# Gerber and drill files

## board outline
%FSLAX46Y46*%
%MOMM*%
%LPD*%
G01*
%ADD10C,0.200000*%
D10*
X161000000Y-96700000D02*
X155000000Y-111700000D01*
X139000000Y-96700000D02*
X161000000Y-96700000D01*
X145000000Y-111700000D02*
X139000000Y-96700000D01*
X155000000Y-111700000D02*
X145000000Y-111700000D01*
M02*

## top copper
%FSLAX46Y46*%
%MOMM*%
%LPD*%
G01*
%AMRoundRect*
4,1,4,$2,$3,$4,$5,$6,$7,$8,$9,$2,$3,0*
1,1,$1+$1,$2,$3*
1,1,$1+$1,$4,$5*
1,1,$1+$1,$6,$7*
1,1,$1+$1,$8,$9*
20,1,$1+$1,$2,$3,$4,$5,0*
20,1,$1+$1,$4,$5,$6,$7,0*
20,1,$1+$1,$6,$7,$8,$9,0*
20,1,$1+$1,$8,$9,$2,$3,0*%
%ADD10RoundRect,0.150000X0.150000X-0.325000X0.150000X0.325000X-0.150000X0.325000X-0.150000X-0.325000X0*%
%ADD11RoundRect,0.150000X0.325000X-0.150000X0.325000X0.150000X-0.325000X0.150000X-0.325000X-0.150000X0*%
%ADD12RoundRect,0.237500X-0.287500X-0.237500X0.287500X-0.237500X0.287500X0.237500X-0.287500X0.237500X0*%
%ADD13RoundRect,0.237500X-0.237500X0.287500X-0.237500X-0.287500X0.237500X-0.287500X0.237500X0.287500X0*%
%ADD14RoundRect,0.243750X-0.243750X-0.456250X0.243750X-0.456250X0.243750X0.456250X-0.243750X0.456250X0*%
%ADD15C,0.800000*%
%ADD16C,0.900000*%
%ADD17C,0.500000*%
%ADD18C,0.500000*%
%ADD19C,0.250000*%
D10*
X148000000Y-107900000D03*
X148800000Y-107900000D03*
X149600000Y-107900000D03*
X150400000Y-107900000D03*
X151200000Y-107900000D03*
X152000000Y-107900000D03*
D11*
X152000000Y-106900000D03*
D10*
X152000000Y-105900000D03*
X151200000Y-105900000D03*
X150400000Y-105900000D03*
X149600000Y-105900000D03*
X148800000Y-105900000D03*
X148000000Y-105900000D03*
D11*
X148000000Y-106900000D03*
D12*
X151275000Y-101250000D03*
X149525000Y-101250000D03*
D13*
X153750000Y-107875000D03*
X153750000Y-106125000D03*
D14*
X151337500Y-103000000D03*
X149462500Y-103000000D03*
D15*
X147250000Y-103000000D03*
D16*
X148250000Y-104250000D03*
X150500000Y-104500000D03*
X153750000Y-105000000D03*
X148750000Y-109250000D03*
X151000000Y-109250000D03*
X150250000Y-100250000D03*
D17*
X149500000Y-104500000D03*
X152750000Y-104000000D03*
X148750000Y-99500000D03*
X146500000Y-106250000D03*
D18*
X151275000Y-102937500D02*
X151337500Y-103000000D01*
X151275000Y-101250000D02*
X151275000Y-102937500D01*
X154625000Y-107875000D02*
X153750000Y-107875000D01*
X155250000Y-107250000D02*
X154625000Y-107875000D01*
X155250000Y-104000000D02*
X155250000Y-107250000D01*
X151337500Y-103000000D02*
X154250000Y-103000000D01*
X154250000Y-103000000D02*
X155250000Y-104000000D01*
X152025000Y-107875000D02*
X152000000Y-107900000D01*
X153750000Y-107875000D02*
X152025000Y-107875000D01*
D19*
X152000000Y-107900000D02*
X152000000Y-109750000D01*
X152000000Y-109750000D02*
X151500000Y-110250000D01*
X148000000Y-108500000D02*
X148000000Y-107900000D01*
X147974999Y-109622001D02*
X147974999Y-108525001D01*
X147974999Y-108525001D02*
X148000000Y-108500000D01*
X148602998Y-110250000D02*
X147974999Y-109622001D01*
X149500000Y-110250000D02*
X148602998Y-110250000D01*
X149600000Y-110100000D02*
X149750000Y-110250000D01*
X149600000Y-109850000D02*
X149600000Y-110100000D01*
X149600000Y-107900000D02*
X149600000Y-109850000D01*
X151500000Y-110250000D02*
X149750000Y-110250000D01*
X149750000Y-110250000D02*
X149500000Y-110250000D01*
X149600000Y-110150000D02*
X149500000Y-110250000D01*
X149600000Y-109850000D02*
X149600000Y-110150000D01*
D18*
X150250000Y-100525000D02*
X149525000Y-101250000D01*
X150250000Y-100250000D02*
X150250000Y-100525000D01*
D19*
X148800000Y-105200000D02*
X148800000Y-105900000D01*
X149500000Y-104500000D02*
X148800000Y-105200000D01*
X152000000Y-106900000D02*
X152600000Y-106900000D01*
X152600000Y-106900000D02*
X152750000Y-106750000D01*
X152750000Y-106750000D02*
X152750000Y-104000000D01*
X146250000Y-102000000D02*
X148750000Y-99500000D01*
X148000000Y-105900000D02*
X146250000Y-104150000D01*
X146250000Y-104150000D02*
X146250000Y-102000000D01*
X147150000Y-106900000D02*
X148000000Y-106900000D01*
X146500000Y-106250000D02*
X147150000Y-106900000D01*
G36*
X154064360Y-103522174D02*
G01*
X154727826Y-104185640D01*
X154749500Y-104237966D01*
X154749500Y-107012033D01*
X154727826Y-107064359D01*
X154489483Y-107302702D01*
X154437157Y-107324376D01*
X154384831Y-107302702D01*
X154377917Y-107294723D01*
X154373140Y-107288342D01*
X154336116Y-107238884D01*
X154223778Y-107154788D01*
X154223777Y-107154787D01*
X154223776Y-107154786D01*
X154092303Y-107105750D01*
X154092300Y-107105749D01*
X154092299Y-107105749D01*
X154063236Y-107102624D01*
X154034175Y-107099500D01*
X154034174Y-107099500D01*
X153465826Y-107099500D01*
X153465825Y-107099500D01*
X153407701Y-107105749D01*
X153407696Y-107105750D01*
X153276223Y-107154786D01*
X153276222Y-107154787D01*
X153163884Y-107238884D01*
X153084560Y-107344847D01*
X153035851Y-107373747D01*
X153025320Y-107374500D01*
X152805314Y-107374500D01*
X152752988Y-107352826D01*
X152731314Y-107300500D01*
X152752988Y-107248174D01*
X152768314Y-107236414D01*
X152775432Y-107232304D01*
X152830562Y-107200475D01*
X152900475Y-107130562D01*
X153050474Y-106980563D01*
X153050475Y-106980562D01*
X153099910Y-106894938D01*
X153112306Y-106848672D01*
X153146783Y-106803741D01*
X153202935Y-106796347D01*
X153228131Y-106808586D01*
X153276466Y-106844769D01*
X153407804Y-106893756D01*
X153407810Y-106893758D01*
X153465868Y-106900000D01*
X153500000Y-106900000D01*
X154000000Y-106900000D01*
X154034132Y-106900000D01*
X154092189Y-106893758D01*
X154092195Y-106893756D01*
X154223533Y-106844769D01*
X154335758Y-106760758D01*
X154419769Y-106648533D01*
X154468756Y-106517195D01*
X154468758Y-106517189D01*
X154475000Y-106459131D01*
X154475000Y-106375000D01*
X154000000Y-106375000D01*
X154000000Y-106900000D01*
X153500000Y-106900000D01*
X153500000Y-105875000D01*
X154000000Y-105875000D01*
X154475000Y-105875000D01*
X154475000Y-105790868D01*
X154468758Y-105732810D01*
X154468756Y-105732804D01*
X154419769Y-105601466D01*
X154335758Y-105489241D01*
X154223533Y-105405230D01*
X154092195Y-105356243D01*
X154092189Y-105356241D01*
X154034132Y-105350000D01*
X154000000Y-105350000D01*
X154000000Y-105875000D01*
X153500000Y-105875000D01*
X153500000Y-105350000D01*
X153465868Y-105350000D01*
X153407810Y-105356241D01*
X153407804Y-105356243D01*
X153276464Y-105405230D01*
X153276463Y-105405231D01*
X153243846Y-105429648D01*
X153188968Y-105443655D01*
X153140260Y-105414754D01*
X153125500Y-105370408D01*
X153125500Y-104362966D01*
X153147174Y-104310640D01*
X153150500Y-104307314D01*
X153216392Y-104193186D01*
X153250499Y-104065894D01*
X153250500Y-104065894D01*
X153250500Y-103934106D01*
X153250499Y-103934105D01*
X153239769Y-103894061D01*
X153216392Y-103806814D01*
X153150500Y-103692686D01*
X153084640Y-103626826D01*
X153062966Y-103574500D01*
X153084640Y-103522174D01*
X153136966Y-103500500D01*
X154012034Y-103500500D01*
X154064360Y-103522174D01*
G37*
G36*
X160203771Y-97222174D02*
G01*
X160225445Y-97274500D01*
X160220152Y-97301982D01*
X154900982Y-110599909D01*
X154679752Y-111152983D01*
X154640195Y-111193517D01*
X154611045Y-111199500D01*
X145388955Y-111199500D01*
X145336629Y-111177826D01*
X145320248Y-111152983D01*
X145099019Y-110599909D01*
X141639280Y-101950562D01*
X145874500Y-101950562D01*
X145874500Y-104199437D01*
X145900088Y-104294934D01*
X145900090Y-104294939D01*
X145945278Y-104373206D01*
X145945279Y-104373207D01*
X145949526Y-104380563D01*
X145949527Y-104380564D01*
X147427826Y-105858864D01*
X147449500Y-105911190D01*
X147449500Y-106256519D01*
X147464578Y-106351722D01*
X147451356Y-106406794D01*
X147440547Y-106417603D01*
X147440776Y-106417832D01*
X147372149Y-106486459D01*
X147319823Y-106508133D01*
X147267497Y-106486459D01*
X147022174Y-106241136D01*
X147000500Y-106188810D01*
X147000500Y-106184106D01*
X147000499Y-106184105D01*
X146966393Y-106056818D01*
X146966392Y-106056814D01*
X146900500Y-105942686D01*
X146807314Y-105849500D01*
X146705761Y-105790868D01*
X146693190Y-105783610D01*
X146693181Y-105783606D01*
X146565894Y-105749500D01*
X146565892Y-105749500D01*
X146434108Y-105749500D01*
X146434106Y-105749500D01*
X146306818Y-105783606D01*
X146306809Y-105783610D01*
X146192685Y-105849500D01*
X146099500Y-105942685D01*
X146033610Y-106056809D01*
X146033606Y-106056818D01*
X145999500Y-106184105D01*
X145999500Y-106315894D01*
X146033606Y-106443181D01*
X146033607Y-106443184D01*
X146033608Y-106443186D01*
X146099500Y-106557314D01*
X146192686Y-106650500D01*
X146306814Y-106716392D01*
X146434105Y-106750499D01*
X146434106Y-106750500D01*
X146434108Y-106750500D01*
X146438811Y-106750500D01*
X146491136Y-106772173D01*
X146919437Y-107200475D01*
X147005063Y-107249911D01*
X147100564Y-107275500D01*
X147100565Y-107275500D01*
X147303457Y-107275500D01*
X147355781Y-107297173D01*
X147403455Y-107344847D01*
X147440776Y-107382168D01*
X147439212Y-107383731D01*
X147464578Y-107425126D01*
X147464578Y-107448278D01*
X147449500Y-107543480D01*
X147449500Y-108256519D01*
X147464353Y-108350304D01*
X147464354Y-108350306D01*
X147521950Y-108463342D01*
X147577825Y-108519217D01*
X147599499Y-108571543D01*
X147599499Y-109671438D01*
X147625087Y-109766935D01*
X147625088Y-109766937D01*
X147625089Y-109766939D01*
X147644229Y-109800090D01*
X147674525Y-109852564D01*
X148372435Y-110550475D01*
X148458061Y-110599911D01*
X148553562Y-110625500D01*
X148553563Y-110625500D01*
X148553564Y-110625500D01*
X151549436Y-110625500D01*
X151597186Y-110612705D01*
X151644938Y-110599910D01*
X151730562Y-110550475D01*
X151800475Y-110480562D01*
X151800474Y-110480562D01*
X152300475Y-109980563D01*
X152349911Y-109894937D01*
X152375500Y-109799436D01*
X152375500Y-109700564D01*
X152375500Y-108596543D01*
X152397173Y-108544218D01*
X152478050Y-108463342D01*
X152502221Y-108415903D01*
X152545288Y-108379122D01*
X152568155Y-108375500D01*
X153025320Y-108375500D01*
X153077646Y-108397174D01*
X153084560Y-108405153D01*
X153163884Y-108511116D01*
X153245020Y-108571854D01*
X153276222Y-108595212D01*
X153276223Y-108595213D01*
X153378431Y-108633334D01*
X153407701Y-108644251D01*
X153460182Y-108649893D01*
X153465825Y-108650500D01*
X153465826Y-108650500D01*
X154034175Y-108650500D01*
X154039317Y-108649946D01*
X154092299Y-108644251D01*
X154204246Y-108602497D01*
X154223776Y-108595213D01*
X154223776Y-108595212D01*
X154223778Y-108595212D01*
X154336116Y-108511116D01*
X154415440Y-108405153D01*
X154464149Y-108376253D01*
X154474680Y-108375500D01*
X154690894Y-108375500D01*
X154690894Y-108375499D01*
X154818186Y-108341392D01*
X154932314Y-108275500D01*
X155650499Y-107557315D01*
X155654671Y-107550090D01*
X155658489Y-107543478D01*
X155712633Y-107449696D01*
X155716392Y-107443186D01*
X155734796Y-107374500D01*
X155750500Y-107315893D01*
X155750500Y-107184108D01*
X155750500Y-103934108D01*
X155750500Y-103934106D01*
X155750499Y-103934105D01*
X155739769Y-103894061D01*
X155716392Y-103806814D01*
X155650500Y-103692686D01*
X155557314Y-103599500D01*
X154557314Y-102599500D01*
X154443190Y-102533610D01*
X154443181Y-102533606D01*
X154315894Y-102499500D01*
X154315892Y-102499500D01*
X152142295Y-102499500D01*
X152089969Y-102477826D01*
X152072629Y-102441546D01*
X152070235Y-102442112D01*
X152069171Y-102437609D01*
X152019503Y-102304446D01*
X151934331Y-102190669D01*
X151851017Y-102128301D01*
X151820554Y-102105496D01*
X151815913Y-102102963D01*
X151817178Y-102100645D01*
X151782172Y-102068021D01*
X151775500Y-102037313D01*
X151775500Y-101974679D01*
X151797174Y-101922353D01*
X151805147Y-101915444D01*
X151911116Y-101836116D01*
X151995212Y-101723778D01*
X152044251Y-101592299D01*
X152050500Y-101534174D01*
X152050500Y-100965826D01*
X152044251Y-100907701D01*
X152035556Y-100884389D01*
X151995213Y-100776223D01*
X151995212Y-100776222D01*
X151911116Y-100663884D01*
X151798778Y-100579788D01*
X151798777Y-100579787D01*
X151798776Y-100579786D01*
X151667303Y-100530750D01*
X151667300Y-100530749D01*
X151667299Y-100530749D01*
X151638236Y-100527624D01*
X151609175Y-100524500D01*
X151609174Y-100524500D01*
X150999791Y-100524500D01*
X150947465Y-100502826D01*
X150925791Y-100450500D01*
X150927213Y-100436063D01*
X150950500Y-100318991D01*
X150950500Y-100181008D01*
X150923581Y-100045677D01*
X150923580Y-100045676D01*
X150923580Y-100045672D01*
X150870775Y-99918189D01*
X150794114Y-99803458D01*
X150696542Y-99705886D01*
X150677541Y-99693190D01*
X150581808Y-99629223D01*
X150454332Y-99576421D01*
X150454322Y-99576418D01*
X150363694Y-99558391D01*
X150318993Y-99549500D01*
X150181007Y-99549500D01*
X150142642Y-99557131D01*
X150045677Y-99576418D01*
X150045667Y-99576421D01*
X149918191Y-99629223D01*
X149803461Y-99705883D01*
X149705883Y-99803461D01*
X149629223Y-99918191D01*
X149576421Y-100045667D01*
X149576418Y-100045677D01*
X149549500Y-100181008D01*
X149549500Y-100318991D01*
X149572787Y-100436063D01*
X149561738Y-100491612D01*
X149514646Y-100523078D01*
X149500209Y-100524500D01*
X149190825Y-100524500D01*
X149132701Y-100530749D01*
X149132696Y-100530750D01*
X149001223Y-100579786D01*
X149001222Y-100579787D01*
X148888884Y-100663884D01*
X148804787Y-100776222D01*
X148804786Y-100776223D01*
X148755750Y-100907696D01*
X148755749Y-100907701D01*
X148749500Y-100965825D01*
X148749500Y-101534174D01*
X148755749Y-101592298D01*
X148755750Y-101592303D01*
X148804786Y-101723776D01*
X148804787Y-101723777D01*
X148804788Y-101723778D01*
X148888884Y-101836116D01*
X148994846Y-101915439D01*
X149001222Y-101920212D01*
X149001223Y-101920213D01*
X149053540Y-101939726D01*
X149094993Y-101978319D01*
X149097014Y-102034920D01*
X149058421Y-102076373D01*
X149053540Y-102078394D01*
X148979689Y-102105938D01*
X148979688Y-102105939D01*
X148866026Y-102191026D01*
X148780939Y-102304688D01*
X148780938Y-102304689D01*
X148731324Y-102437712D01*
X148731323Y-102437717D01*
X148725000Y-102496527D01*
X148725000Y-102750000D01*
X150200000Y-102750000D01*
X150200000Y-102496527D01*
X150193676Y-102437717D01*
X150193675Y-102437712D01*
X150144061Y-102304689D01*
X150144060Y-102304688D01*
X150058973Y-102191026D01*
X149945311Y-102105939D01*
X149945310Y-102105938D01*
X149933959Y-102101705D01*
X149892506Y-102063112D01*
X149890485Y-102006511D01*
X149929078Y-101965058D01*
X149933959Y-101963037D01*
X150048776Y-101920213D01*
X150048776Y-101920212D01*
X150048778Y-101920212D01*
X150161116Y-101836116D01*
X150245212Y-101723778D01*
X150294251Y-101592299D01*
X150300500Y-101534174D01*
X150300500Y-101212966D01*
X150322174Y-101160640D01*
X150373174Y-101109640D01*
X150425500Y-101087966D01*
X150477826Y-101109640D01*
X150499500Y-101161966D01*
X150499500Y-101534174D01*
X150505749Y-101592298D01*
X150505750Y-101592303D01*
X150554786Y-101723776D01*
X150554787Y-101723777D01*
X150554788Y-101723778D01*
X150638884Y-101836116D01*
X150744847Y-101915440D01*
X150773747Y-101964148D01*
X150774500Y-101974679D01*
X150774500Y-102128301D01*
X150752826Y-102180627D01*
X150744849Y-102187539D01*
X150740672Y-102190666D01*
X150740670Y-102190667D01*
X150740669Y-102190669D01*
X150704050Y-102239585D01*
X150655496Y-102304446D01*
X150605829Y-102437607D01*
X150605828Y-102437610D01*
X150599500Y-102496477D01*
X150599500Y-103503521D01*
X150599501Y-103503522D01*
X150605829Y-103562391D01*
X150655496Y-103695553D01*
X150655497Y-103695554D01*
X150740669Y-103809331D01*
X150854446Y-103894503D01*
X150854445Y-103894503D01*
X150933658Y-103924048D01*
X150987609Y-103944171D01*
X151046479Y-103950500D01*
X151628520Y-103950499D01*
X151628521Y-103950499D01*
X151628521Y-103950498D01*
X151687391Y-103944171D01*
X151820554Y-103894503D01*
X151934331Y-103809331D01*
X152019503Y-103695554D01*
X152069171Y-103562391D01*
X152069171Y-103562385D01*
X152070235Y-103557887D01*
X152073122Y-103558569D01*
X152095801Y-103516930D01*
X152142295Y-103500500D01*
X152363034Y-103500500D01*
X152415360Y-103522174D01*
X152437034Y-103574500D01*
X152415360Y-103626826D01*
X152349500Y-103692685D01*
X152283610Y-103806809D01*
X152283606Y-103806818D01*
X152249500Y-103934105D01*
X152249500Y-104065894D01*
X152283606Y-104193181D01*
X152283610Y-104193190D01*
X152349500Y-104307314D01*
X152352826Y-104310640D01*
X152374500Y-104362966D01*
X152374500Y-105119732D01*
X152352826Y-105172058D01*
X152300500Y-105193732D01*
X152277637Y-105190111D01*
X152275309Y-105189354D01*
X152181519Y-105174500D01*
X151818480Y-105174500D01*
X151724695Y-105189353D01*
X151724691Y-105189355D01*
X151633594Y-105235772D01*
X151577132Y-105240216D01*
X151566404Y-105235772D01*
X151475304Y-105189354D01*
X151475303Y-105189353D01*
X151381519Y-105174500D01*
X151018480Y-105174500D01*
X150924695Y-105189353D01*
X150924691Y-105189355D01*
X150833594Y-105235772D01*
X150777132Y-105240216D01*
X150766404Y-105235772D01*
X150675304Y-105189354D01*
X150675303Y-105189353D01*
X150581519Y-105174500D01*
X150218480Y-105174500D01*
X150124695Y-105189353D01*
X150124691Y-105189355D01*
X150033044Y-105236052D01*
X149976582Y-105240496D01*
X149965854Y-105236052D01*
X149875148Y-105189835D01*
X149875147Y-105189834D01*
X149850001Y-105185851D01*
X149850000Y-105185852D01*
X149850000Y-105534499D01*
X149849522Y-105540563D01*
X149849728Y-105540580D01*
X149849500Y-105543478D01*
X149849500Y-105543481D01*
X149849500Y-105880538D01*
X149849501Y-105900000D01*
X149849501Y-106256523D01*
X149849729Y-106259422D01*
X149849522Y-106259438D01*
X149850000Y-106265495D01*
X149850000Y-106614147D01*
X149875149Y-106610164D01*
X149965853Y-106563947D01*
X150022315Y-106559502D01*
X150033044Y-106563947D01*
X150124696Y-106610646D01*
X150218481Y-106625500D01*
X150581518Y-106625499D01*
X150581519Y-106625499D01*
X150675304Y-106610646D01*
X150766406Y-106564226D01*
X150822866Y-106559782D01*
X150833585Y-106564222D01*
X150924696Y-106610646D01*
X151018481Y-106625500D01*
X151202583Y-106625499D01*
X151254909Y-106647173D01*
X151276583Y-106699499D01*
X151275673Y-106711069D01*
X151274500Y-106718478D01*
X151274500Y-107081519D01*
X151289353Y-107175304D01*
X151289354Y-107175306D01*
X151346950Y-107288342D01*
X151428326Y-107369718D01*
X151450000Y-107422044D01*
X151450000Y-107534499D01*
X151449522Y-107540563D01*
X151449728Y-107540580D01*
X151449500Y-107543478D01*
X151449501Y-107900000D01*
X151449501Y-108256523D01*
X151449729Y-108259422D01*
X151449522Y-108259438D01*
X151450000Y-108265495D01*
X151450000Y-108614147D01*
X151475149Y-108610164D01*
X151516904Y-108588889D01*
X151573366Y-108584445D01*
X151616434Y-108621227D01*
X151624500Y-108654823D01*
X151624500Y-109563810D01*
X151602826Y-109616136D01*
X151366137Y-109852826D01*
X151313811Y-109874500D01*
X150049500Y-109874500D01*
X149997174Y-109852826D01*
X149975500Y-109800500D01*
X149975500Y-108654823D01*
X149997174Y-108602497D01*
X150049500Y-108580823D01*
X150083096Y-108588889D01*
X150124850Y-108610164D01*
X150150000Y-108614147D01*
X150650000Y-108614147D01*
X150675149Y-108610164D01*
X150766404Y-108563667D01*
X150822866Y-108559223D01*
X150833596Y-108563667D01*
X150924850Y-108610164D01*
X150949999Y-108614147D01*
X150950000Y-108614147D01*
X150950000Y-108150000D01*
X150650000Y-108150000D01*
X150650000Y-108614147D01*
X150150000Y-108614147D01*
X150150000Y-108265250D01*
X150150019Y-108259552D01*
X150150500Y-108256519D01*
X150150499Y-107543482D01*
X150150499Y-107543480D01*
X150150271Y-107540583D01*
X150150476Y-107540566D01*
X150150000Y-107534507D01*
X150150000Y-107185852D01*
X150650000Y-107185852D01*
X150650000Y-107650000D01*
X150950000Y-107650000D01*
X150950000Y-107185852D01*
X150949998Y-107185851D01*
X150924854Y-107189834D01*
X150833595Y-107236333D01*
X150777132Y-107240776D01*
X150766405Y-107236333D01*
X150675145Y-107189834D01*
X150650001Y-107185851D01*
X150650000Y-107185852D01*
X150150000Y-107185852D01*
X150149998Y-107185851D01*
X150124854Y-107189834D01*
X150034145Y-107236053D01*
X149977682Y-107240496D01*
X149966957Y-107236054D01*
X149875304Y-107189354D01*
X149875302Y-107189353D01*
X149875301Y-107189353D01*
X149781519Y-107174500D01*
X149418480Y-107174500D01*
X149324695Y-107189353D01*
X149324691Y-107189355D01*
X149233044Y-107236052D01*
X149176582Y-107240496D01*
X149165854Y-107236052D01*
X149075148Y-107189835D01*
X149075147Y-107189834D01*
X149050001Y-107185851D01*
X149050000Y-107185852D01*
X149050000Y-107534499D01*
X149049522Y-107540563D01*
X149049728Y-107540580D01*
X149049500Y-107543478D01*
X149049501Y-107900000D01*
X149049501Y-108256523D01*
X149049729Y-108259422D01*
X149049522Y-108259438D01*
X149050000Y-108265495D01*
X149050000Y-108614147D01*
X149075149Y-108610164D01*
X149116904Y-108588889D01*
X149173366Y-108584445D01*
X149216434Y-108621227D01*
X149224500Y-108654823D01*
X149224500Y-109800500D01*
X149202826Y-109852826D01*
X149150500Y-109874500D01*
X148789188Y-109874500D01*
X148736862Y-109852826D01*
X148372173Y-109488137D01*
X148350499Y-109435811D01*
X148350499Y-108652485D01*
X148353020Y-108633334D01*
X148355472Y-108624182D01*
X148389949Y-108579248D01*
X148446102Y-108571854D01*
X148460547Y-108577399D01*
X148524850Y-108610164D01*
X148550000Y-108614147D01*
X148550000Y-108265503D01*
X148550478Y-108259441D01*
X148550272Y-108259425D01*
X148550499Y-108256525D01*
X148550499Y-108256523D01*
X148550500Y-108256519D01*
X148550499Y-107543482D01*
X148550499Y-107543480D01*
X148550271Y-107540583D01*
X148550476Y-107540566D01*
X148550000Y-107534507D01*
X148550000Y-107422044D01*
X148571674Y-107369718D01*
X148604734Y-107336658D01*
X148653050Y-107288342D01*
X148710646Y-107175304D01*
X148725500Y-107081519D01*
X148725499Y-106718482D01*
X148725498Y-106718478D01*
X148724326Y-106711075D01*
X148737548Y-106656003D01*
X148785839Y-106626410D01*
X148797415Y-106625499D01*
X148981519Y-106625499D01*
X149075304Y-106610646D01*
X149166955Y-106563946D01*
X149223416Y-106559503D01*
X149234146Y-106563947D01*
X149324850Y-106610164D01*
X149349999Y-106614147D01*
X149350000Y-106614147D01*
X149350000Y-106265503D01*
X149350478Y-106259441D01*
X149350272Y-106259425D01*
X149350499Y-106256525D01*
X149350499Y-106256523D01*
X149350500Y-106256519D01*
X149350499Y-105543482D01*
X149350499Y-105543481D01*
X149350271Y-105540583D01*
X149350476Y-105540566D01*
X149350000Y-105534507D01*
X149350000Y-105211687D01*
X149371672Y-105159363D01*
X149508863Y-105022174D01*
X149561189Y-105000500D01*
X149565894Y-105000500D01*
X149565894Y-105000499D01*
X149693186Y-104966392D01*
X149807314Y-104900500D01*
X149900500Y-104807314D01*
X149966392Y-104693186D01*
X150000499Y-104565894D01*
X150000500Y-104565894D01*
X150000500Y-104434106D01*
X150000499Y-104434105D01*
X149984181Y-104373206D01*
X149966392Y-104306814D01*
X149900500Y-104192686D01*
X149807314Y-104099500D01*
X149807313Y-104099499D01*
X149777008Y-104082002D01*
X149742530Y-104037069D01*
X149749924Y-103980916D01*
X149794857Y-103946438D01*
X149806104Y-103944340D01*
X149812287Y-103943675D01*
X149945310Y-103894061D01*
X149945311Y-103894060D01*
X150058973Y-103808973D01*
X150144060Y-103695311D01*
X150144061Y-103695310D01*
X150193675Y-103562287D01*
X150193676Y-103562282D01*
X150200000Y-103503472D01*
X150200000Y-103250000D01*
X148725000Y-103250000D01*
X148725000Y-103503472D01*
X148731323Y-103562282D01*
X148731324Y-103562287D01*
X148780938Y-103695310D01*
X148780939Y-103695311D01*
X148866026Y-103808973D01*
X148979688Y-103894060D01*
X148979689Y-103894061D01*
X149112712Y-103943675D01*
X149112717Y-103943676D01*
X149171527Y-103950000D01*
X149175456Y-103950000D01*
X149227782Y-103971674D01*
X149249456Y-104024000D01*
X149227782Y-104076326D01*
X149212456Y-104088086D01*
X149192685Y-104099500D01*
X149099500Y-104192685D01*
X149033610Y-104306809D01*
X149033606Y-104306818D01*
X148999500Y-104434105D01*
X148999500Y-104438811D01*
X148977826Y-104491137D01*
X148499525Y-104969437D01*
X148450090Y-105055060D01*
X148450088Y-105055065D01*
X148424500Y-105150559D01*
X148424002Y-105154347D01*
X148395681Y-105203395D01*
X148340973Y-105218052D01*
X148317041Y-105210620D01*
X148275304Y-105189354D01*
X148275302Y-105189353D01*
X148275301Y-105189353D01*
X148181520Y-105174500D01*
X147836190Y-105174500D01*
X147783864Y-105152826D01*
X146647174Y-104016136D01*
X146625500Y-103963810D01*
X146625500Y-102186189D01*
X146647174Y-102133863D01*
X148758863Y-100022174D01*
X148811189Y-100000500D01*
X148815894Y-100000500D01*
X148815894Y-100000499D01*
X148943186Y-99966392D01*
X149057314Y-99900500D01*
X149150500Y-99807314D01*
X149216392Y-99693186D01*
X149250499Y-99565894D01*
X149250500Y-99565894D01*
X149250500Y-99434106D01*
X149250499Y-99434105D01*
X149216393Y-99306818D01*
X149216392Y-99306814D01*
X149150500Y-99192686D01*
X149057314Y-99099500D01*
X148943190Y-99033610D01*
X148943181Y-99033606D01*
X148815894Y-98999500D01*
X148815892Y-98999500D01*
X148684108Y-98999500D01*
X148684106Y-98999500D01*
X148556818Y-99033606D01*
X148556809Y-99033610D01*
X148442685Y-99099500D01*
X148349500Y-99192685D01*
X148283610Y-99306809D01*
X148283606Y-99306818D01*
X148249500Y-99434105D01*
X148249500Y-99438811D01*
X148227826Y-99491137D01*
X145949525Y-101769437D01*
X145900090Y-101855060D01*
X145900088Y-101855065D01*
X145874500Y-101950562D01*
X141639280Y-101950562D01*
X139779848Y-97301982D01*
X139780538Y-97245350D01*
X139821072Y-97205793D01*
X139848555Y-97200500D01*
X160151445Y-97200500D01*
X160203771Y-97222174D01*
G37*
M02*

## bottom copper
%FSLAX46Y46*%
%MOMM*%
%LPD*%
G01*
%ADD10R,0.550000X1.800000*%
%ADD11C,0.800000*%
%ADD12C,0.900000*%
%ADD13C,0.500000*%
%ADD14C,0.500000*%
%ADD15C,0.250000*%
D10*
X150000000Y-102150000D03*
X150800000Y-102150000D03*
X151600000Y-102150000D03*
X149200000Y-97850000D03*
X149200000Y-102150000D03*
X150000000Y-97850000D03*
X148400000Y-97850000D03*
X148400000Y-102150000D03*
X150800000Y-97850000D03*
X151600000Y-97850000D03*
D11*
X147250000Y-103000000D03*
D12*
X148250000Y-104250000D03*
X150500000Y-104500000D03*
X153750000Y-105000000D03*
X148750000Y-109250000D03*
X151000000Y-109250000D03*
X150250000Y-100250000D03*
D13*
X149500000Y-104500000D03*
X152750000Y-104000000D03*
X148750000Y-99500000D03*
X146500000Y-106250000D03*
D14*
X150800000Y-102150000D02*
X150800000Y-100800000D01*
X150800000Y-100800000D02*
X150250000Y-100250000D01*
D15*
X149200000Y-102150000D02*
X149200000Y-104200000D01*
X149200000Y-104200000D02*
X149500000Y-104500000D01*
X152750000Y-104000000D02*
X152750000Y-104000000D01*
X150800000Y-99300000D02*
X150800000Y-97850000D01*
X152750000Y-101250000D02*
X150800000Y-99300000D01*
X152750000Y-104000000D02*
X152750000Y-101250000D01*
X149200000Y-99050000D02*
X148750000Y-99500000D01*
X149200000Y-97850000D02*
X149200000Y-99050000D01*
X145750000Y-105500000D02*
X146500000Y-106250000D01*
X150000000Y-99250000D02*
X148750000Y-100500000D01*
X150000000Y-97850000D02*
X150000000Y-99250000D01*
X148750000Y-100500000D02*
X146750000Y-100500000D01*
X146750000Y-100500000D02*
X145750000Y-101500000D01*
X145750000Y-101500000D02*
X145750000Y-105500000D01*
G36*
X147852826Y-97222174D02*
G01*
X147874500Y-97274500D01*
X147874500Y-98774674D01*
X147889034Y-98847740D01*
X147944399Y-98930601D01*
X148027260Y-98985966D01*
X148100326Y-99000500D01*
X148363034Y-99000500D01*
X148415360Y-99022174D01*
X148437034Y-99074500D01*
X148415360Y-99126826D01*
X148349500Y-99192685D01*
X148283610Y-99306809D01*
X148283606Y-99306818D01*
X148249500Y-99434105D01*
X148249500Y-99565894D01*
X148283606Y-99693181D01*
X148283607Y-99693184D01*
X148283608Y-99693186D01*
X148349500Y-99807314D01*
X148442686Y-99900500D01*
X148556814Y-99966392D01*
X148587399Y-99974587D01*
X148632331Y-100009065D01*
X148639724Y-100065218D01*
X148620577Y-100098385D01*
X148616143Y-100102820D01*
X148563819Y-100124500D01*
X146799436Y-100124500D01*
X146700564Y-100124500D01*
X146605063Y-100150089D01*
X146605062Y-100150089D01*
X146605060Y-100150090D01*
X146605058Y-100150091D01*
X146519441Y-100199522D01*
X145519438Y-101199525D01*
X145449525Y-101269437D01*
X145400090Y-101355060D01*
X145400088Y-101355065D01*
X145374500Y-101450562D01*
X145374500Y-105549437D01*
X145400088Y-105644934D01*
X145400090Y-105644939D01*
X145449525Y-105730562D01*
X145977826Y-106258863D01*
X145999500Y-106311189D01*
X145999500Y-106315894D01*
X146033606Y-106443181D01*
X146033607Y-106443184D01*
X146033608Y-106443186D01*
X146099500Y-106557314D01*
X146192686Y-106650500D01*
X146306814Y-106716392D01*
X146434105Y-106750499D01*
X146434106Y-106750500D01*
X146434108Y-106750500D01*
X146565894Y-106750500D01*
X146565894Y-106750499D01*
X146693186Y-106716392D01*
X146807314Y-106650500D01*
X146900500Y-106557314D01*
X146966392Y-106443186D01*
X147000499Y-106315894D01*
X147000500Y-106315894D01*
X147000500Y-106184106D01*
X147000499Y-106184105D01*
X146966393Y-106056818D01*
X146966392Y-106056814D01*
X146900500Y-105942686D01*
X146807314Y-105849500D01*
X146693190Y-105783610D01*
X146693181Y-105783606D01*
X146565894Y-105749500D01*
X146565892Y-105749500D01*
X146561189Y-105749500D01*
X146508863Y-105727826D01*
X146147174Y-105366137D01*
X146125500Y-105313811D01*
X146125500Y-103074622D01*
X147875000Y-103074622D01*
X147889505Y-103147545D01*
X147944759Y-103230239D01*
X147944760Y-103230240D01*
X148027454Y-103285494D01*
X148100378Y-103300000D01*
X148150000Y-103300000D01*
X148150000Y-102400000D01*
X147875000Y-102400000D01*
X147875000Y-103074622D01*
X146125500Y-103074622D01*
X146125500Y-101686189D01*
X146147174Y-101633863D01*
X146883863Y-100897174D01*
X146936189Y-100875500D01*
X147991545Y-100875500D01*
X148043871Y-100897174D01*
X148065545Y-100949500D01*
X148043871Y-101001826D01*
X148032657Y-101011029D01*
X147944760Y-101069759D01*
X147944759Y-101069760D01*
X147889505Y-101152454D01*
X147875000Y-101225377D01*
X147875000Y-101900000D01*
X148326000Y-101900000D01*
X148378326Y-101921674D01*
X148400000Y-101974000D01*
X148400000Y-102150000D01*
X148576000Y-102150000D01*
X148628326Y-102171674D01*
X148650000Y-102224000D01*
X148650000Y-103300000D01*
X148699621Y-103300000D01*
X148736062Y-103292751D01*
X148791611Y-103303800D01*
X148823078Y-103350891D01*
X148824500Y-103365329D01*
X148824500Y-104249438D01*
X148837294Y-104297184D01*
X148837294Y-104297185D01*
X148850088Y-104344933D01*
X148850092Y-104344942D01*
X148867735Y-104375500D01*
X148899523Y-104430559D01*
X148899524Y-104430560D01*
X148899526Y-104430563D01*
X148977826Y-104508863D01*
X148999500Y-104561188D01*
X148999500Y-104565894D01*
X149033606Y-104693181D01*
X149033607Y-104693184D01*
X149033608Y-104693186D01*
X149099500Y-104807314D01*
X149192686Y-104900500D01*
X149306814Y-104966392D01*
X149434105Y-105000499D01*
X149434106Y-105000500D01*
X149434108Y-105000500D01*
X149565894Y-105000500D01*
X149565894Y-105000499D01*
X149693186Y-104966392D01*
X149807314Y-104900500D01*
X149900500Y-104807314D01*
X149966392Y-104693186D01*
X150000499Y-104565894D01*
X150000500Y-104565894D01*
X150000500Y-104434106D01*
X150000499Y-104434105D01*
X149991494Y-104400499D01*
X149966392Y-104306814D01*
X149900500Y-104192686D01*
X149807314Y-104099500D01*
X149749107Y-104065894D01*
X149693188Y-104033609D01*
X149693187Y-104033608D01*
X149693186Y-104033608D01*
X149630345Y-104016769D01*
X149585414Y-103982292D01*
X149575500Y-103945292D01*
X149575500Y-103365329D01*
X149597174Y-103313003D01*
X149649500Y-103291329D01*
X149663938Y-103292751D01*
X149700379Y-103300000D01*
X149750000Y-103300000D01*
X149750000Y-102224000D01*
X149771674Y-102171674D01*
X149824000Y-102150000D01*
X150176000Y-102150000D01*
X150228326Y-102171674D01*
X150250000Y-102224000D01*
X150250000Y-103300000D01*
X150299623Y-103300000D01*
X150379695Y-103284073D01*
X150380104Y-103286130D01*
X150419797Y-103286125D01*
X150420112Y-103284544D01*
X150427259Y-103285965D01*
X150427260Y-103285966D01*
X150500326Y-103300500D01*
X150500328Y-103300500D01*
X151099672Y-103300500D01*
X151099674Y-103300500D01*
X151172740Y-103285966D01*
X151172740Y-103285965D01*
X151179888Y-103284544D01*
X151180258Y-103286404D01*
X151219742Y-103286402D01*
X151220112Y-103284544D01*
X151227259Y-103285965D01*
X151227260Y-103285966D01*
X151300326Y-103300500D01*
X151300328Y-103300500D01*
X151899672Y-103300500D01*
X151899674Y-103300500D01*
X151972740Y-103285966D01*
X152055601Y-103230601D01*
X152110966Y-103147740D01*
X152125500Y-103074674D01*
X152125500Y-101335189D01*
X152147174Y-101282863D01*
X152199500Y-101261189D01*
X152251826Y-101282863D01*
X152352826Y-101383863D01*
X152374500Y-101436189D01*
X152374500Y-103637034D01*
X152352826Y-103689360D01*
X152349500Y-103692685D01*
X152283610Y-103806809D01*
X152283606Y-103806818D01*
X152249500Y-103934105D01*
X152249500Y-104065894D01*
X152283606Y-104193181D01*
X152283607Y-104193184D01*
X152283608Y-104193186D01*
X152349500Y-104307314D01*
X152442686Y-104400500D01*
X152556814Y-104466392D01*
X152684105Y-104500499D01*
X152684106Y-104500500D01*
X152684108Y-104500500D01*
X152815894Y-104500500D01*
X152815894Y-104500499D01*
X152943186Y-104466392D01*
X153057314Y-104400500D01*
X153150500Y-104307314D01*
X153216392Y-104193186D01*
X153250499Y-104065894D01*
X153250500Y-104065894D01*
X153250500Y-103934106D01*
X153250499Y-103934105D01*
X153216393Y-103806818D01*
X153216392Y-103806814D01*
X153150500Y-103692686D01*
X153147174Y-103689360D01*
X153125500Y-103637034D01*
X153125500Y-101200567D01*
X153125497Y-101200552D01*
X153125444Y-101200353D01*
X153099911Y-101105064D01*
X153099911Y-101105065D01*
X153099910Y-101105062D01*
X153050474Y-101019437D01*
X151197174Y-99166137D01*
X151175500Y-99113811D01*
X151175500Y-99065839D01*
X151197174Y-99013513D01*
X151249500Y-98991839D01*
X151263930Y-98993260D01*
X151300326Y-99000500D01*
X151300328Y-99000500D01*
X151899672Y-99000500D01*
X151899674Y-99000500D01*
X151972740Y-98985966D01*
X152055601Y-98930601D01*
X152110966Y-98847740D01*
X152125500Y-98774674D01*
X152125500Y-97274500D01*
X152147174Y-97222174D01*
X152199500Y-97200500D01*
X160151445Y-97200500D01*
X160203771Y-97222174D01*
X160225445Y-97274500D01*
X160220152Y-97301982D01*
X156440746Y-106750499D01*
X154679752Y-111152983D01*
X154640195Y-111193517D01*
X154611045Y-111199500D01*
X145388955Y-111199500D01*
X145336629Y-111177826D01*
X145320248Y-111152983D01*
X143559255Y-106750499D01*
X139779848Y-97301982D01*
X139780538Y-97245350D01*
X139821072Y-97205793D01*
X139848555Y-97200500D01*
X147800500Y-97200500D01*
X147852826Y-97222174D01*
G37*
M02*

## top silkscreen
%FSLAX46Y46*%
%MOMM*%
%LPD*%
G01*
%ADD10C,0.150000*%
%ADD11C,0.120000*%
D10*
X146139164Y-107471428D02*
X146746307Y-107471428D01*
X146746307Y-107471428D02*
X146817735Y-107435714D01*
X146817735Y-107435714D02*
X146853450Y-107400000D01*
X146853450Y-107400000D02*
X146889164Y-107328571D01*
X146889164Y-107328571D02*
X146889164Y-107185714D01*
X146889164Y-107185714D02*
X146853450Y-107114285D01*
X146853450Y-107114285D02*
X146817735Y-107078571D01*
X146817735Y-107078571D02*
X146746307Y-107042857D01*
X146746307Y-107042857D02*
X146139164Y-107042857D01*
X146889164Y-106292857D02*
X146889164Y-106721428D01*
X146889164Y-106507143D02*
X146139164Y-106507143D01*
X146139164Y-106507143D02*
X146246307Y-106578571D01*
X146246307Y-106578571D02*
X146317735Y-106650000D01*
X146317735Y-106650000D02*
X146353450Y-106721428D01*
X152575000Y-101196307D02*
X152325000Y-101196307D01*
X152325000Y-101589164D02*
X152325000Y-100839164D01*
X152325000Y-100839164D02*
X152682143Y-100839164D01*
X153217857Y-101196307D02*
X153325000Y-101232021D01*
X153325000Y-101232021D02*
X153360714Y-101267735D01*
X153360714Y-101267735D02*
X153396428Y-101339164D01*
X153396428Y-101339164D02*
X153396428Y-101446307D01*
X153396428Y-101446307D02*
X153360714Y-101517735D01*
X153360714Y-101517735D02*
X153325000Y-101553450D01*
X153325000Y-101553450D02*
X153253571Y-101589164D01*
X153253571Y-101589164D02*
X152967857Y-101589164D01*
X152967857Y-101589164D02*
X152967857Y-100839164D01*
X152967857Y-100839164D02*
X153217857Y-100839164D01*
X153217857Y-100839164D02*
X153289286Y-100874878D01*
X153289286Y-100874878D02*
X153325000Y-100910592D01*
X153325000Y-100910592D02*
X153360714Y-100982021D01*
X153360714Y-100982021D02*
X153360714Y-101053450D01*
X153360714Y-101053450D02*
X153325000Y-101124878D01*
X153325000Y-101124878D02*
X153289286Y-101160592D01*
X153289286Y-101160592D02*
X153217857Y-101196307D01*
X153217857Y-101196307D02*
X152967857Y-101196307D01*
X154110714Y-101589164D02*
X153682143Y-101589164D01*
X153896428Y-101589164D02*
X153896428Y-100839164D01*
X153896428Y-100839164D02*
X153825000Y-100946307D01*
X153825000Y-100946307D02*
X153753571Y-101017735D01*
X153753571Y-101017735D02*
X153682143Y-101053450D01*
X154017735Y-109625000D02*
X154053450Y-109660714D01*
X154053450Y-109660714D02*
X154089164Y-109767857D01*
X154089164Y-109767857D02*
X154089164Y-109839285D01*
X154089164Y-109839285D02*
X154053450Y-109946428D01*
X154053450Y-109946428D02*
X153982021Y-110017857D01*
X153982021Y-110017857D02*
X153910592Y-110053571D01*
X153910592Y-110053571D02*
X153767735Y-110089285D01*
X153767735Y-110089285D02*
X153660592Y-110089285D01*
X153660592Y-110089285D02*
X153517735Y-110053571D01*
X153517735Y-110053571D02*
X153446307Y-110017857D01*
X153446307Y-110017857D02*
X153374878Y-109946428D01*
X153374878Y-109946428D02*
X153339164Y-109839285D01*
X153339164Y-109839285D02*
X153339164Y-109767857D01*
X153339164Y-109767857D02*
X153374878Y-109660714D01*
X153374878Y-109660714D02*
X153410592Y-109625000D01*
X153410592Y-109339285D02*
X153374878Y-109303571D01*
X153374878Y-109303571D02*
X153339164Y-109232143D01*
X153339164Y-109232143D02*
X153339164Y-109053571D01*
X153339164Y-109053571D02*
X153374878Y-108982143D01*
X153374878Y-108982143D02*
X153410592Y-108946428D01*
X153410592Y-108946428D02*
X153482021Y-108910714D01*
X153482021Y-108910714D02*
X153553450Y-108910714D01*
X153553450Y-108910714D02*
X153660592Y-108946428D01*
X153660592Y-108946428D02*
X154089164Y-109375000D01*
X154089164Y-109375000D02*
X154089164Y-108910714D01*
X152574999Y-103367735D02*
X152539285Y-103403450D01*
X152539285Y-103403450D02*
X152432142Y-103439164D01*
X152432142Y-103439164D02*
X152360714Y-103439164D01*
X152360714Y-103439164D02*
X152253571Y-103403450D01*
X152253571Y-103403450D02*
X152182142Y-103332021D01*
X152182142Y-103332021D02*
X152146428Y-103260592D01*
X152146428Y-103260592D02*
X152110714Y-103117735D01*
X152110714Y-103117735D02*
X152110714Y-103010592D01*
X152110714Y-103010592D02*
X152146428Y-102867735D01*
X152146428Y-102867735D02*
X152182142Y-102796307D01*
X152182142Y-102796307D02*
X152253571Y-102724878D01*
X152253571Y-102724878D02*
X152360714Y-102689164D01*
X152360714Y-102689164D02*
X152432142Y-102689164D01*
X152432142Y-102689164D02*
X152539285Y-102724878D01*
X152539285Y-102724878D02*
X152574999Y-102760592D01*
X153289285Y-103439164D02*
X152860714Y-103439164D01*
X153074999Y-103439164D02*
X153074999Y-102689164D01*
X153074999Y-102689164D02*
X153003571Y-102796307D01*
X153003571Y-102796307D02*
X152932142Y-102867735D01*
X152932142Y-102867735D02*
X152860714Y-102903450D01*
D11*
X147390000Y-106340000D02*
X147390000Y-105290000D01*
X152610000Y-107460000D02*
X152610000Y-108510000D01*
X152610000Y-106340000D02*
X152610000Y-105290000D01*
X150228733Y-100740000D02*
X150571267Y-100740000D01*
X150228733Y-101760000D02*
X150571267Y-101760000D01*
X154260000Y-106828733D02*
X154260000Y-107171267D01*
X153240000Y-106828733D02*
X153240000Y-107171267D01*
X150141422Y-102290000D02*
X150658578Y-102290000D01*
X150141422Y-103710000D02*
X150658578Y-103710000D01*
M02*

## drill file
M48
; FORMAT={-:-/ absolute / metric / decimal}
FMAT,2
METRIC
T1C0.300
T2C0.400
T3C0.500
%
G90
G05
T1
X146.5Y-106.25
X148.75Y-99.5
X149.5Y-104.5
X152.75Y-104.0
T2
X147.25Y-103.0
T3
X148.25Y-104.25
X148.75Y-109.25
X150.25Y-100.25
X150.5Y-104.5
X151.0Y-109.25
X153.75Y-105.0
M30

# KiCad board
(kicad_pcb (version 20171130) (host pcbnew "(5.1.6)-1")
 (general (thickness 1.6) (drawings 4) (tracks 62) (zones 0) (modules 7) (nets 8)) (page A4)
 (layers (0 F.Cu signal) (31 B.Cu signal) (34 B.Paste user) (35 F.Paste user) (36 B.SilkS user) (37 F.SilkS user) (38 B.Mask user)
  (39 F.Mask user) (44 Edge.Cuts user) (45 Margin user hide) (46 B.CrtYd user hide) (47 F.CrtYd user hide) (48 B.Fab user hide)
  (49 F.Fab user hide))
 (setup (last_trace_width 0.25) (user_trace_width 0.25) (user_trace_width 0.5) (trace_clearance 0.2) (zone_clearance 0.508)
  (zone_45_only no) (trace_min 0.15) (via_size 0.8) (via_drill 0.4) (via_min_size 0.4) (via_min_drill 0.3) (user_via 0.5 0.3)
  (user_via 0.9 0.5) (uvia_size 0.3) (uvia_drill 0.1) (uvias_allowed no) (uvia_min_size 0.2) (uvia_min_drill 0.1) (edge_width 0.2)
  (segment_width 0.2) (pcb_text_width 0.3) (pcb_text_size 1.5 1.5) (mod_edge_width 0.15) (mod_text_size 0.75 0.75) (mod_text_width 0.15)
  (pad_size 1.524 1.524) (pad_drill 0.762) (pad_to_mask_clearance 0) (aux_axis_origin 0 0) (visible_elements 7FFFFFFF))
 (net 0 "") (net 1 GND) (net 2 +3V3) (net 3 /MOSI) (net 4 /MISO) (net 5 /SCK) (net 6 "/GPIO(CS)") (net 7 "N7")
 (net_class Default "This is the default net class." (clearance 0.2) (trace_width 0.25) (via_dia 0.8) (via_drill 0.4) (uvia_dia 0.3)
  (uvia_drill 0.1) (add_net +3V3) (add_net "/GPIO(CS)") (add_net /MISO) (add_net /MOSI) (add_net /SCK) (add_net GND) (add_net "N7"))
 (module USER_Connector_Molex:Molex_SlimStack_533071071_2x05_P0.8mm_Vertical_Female (layer B.Cu) (at 150 100 180)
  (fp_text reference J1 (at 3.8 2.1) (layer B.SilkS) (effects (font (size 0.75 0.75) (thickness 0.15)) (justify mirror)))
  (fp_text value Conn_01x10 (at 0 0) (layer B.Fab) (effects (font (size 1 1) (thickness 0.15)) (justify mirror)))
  (pad 5 smd rect (at 0 -2.15) (size 0.55 1.8) (layers B.Cu B.Paste B.Mask) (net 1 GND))
  (pad 3 smd rect (at -0.8 -2.15) (size 0.55 1.8) (layers B.Cu B.Paste B.Mask) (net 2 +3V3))
  (pad 1 smd rect (at -1.6 -2.15) (size 0.55 1.8) (layers B.Cu B.Paste B.Mask))
  (pad 8 smd rect (at 0.8 2.15) (size 0.55 1.8) (layers B.Cu B.Paste B.Mask) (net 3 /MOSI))
  (pad 7 smd rect (at 0.8 -2.15) (size 0.55 1.8) (layers B.Cu B.Paste B.Mask) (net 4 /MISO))
  (pad 6 smd rect (at 0 2.15) (size 0.55 1.8) (layers B.Cu B.Paste B.Mask) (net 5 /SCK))
  (pad 10 smd rect (at 1.6 2.15) (size 0.55 1.8) (layers B.Cu B.Paste B.Mask))
  (pad 9 smd rect (at 1.6 -2.15) (size 0.55 1.8) (layers B.Cu B.Paste B.Mask) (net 1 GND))
  (pad 4 smd rect (at -0.8 2.15) (size 0.55 1.8) (layers B.Cu B.Paste B.Mask) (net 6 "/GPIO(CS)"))
  (pad 2 smd rect (at -1.6 2.15) (size 0.55 1.8) (layers B.Cu B.Paste B.Mask)))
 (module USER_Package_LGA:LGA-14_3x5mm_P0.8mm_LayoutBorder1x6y (layer F.Cu) (at 150 106.9 90)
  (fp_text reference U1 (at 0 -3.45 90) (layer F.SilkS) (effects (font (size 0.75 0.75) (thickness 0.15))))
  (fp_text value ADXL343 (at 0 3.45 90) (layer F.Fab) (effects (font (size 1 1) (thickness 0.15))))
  (fp_line (start 0.56 -2.61) (end 1.61 -2.61) (layer F.SilkS) (width 0.12))
  (fp_line (start -0.56 2.61) (end -1.61 2.61) (layer F.SilkS) (width 0.12))
  (fp_line (start 0.56 2.61) (end 1.61 2.61) (layer F.SilkS) (width 0.12))
  (pad 1 smd roundrect (at -1 -2 90) (size 0.95 0.6) (layers F.Cu F.Paste F.Mask) (roundrect_rratio 0.25) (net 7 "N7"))
  (pad 2 smd roundrect (at -1 -1.2 90) (size 0.95 0.6) (layers F.Cu F.Paste F.Mask) (roundrect_rratio 0.25) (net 1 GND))
  (pad 3 smd roundrect (at -1 -0.4 90) (size 0.95 0.6) (layers F.Cu F.Paste F.Mask) (roundrect_rratio 0.25) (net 7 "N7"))
  (pad 4 smd roundrect (at -1 0.4 90) (size 0.95 0.6) (layers F.Cu F.Paste F.Mask) (roundrect_rratio 0.25) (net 1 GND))
  (pad 5 smd roundrect (at -1 1.2 90) (size 0.95 0.6) (layers F.Cu F.Paste F.Mask) (roundrect_rratio 0.25) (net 1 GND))
  (pad 6 smd roundrect (at -1 2 90) (size 0.95 0.6) (layers F.Cu F.Paste F.Mask) (roundrect_rratio 0.25) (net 7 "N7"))
  (pad 7 smd roundrect (at 0 2 90) (size 0.6 0.95) (layers F.Cu F.Paste F.Mask) (roundrect_rratio 0.25) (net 6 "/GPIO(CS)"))
  (pad 8 smd roundrect (at 1 2 90) (size 0.95 0.6) (layers F.Cu F.Paste F.Mask) (roundrect_rratio 0.25))
  (pad 9 smd roundrect (at 1 1.2 90) (size 0.95 0.6) (layers F.Cu F.Paste F.Mask) (roundrect_rratio 0.25))
  (pad 10 smd roundrect (at 1 0.4 90) (size 0.95 0.6) (layers F.Cu F.Paste F.Mask) (roundrect_rratio 0.25))
  (pad 11 smd roundrect (at 1 -0.4 90) (size 0.95 0.6) (layers F.Cu F.Paste F.Mask) (roundrect_rratio 0.25) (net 1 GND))
  (pad 12 smd roundrect (at 1 -1.2 90) (size 0.95 0.6) (layers F.Cu F.Paste F.Mask) (roundrect_rratio 0.25) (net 4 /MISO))
  (pad 13 smd roundrect (at 1 -2 90) (size 0.95 0.6) (layers F.Cu F.Paste F.Mask) (roundrect_rratio 0.25) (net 3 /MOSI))
  (pad 14 smd roundrect (at 0 -2 90) (size 0.6 0.95) (layers F.Cu F.Paste F.Mask) (roundrect_rratio 0.25) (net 5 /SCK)))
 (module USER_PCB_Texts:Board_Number (layer B.Cu) (at 145.5 108.8)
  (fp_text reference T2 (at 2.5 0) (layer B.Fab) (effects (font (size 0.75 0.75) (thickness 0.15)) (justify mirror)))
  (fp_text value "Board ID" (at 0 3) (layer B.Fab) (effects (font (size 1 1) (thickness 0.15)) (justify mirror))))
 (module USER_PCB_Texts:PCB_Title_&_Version (layer F.Cu) (at 147.594999 110.734999)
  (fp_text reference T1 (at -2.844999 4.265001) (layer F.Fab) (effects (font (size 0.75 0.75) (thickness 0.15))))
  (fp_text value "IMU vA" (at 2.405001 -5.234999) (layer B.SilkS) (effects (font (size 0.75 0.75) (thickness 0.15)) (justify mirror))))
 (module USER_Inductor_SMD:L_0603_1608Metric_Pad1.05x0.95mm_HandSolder (layer F.Cu) (at 150.4 101.25)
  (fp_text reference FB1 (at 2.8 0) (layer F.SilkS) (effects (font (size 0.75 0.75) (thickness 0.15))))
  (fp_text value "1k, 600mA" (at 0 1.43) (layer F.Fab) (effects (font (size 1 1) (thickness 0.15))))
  (fp_line (start -0.171267 -0.51) (end 0.171267 -0.51) (layer F.SilkS) (width 0.12))
  (fp_line (start -0.171267 0.51) (end 0.171267 0.51) (layer F.SilkS) (width 0.12))
  (pad 2 smd roundrect (at 0.875 0) (size 1.05 0.95) (layers F.Cu F.Paste F.Mask) (roundrect_rratio 0.25) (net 7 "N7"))
  (pad 1 smd roundrect (at -0.875 0) (size 1.05 0.95) (layers F.Cu F.Paste F.Mask) (roundrect_rratio 0.25) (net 2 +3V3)))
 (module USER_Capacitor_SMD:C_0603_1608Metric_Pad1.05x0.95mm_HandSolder (layer F.Cu) (at 153.75 107 270)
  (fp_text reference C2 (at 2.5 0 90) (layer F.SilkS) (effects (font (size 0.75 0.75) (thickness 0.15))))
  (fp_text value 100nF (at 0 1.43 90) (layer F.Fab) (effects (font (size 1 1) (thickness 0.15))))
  (fp_line (start -0.171267 -0.51) (end 0.171267 -0.51) (layer F.SilkS) (width 0.12))
  (fp_line (start -0.171267 0.51) (end 0.171267 0.51) (layer F.SilkS) (width 0.12))
  (pad 2 smd roundrect (at 0.875 0 270) (size 1.05 0.95) (layers F.Cu F.Paste F.Mask) (roundrect_rratio 0.25) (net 7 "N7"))
  (pad 1 smd roundrect (at -0.875 0 270) (size 1.05 0.95) (layers F.Cu F.Paste F.Mask) (roundrect_rratio 0.25) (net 1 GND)))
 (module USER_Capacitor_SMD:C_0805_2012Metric (layer F.Cu) (at 150.4 103)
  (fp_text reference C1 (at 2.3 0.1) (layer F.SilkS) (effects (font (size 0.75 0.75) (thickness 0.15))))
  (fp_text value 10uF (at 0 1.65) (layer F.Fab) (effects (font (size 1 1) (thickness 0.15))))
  (fp_line (start -0.258578 -0.71) (end 0.258578 -0.71) (layer F.SilkS) (width 0.12))
  (fp_line (start -0.258578 0.71) (end 0.258578 0.71) (layer F.SilkS) (width 0.12))
  (pad 2 smd roundrect (at 0.9375 0) (size 0.975 1.4) (layers F.Cu F.Paste F.Mask) (roundrect_rratio 0.25) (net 7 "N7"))
  (pad 1 smd roundrect (at -0.9375 0) (size 0.975 1.4) (layers F.Cu F.Paste F.Mask) (roundrect_rratio 0.25) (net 1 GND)))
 (gr_line (start 161 96.7) (end 155 111.7) (layer Edge.Cuts) (width 0.2))
 (gr_line (start 139 96.7) (end 161 96.7) (layer Edge.Cuts) (width 0.2))
 (gr_line (start 145 111.7) (end 139 96.7) (layer Edge.Cuts) (width 0.2))
 (gr_line (start 155 111.7) (end 145 111.7) (layer Edge.Cuts) (width 0.2))
 (segment (start 151.275 102.9375) (end 151.3375 103) (width 0.5) (layer F.Cu) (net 7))
 (segment (start 151.275 101.25) (end 151.275 102.9375) (width 0.5) (layer F.Cu) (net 7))
 (segment (start 154.625 107.875) (end 153.75 107.875) (width 0.5) (layer F.Cu) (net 7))
 (segment (start 155.25 107.25) (end 154.625 107.875) (width 0.5) (layer F.Cu) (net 7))
 (segment (start 155.25 104) (end 155.25 107.25) (width 0.5) (layer F.Cu) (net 7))
 (segment (start 151.3375 103) (end 154.25 103) (width 0.5) (layer F.Cu) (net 7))
 (segment (start 154.25 103) (end 155.25 104) (width 0.5) (layer F.Cu) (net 7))
 (segment (start 152.025 107.875) (end 152 107.9) (width 0.5) (layer F.Cu) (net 7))
 (segment (start 153.75 107.875) (end 152.025 107.875) (width 0.5) (layer F.Cu) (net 7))
 (segment (start 152 107.9) (end 152 109.75) (width 0.25) (layer F.Cu) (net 7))
 (segment (start 152 109.75) (end 151.5 110.25) (width 0.25) (layer F.Cu) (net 7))
 (segment (start 148 108.5) (end 148 107.9) (width 0.25) (layer F.Cu) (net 7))
 (segment (start 147.974999 109.622001) (end 147.974999 108.525001) (width 0.25) (layer F.Cu) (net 7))
 (segment (start 147.974999 108.525001) (end 148 108.5) (width 0.25) (layer F.Cu) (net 7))
 (segment (start 148.602998 110.25) (end 147.974999 109.622001) (width 0.25) (layer F.Cu) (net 7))
 (segment (start 149.5 110.25) (end 148.602998 110.25) (width 0.25) (layer F.Cu) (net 7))
 (segment (start 149.6 110.1) (end 149.75 110.25) (width 0.25) (layer F.Cu) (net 7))
 (segment (start 149.6 109.85) (end 149.6 110.1) (width 0.25) (layer F.Cu) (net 7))
 (segment (start 149.6 107.9) (end 149.6 109.85) (width 0.25) (layer F.Cu) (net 7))
 (segment (start 151.5 110.25) (end 149.75 110.25) (width 0.25) (layer F.Cu) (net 7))
 (segment (start 149.75 110.25) (end 149.5 110.25) (width 0.25) (layer F.Cu) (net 7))
 (segment (start 149.6 110.15) (end 149.5 110.25) (width 0.25) (layer F.Cu) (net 7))
 (segment (start 149.6 109.85) (end 149.6 110.15) (width 0.25) (layer F.Cu) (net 7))
 (via (at 147.25 103) (size 0.8) (drill 0.4) (layers F.Cu B.Cu) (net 1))
 (via (at 148.25 104.25) (size 0.9) (drill 0.5) (layers F.Cu B.Cu) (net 1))
 (via (at 150.5 104.5) (size 0.9) (drill 0.5) (layers F.Cu B.Cu) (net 1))
 (via (at 153.75 105) (size 0.9) (drill 0.5) (layers F.Cu B.Cu) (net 1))
 (via (at 148.75 109.25) (size 0.9) (drill 0.5) (layers F.Cu B.Cu) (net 1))
 (via (at 151 109.25) (size 0.9) (drill 0.5) (layers F.Cu B.Cu) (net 1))
 (segment (start 150.8 102.15) (end 150.8 100.8) (width 0.5) (layer B.Cu) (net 2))
 (via (at 150.25 100.25) (size 0.9) (drill 0.5) (layers F.Cu B.Cu) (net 2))
 (segment (start 150.8 100.8) (end 150.25 100.25) (width 0.5) (layer B.Cu) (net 2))
 (segment (start 150.25 100.525) (end 149.525 101.25) (width 0.5) (layer F.Cu) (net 2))
 (segment (start 150.25 100.25) (end 150.25 100.525) (width 0.5) (layer F.Cu) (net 2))
 (via (at 149.5 104.5) (size 0.5) (drill 0.3) (layers F.Cu B.Cu) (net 4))
 (segment (start 149.2 102.15) (end 149.2 104.2) (width 0.25) (layer B.Cu) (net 4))
 (segment (start 149.2 104.2) (end 149.5 104.5) (width 0.25) (layer B.Cu) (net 4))
 (segment (start 148.8 105.2) (end 148.8 105.9) (width 0.25) (layer F.Cu) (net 4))
 (segment (start 149.5 104.5) (end 148.8 105.2) (width 0.25) (layer F.Cu) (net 4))
 (segment (start 152 106.9) (end 152.6 106.9) (width 0.25) (layer F.Cu) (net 6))
 (segment (start 152.6 106.9) (end 152.75 106.75) (width 0.25) (layer F.Cu) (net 6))
 (segment (start 152.75 106.75) (end 152.75 104) (width 0.25) (layer F.Cu) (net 6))
 (segment (start 152.75 104) (end 152.75 104) (width 0.25) (layer B.Cu) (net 6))
 (segment (start 150.8 99.3) (end 150.8 97.85) (width 0.25) (layer B.Cu) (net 6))
 (segment (start 152.75 101.25) (end 150.8 99.3) (width 0.25) (layer B.Cu) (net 6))
 (segment (start 152.75 104) (end 152.75 101.25) (width 0.25) (layer B.Cu) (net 6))
 (via (at 152.75 104) (size 0.5) (drill 0.3) (layers F.Cu B.Cu) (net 6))
 (segment (start 149.2 99.05) (end 148.75 99.5) (width 0.25) (layer B.Cu) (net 3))
 (segment (start 149.2 97.85) (end 149.2 99.05) (width 0.25) (layer B.Cu) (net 3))
 (segment (start 146.25 102) (end 148.75 99.5) (width 0.25) (layer F.Cu) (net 3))
 (segment (start 148 105.9) (end 146.25 104.15) (width 0.25) (layer F.Cu) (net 3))
 (segment (start 146.25 104.15) (end 146.25 102) (width 0.25) (layer F.Cu) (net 3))
 (via (at 148.75 99.5) (size 0.5) (drill 0.3) (layers F.Cu B.Cu) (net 3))
 (via (at 146.5 106.25) (size 0.5) (drill 0.3) (layers F.Cu B.Cu) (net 5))
 (segment (start 147.15 106.9) (end 148 106.9) (width 0.25) (layer F.Cu) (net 5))
 (segment (start 146.5 106.25) (end 147.15 106.9) (width 0.25) (layer F.Cu) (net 5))
 (segment (start 145.75 105.5) (end 146.5 106.25) (width 0.25) (layer B.Cu) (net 5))
 (segment (start 150 99.25) (end 148.75 100.5) (width 0.25) (layer B.Cu) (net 5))
 (segment (start 150 97.85) (end 150 99.25) (width 0.25) (layer B.Cu) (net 5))
 (segment (start 148.75 100.5) (end 146.75 100.5) (width 0.25) (layer B.Cu) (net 5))
 (segment (start 146.75 100.5) (end 145.75 101.5) (width 0.25) (layer B.Cu) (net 5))
 (segment (start 145.75 101.5) (end 145.75 105.5) (width 0.25) (layer B.Cu) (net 5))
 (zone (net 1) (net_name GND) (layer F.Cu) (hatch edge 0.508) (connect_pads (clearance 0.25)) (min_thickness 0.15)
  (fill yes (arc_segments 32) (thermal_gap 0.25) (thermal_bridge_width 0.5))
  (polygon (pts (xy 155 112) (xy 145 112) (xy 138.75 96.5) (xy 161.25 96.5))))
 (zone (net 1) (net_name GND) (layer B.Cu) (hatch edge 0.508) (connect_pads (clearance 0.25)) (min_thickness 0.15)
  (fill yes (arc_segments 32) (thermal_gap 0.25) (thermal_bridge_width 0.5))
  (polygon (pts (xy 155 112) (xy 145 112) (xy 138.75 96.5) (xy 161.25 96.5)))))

